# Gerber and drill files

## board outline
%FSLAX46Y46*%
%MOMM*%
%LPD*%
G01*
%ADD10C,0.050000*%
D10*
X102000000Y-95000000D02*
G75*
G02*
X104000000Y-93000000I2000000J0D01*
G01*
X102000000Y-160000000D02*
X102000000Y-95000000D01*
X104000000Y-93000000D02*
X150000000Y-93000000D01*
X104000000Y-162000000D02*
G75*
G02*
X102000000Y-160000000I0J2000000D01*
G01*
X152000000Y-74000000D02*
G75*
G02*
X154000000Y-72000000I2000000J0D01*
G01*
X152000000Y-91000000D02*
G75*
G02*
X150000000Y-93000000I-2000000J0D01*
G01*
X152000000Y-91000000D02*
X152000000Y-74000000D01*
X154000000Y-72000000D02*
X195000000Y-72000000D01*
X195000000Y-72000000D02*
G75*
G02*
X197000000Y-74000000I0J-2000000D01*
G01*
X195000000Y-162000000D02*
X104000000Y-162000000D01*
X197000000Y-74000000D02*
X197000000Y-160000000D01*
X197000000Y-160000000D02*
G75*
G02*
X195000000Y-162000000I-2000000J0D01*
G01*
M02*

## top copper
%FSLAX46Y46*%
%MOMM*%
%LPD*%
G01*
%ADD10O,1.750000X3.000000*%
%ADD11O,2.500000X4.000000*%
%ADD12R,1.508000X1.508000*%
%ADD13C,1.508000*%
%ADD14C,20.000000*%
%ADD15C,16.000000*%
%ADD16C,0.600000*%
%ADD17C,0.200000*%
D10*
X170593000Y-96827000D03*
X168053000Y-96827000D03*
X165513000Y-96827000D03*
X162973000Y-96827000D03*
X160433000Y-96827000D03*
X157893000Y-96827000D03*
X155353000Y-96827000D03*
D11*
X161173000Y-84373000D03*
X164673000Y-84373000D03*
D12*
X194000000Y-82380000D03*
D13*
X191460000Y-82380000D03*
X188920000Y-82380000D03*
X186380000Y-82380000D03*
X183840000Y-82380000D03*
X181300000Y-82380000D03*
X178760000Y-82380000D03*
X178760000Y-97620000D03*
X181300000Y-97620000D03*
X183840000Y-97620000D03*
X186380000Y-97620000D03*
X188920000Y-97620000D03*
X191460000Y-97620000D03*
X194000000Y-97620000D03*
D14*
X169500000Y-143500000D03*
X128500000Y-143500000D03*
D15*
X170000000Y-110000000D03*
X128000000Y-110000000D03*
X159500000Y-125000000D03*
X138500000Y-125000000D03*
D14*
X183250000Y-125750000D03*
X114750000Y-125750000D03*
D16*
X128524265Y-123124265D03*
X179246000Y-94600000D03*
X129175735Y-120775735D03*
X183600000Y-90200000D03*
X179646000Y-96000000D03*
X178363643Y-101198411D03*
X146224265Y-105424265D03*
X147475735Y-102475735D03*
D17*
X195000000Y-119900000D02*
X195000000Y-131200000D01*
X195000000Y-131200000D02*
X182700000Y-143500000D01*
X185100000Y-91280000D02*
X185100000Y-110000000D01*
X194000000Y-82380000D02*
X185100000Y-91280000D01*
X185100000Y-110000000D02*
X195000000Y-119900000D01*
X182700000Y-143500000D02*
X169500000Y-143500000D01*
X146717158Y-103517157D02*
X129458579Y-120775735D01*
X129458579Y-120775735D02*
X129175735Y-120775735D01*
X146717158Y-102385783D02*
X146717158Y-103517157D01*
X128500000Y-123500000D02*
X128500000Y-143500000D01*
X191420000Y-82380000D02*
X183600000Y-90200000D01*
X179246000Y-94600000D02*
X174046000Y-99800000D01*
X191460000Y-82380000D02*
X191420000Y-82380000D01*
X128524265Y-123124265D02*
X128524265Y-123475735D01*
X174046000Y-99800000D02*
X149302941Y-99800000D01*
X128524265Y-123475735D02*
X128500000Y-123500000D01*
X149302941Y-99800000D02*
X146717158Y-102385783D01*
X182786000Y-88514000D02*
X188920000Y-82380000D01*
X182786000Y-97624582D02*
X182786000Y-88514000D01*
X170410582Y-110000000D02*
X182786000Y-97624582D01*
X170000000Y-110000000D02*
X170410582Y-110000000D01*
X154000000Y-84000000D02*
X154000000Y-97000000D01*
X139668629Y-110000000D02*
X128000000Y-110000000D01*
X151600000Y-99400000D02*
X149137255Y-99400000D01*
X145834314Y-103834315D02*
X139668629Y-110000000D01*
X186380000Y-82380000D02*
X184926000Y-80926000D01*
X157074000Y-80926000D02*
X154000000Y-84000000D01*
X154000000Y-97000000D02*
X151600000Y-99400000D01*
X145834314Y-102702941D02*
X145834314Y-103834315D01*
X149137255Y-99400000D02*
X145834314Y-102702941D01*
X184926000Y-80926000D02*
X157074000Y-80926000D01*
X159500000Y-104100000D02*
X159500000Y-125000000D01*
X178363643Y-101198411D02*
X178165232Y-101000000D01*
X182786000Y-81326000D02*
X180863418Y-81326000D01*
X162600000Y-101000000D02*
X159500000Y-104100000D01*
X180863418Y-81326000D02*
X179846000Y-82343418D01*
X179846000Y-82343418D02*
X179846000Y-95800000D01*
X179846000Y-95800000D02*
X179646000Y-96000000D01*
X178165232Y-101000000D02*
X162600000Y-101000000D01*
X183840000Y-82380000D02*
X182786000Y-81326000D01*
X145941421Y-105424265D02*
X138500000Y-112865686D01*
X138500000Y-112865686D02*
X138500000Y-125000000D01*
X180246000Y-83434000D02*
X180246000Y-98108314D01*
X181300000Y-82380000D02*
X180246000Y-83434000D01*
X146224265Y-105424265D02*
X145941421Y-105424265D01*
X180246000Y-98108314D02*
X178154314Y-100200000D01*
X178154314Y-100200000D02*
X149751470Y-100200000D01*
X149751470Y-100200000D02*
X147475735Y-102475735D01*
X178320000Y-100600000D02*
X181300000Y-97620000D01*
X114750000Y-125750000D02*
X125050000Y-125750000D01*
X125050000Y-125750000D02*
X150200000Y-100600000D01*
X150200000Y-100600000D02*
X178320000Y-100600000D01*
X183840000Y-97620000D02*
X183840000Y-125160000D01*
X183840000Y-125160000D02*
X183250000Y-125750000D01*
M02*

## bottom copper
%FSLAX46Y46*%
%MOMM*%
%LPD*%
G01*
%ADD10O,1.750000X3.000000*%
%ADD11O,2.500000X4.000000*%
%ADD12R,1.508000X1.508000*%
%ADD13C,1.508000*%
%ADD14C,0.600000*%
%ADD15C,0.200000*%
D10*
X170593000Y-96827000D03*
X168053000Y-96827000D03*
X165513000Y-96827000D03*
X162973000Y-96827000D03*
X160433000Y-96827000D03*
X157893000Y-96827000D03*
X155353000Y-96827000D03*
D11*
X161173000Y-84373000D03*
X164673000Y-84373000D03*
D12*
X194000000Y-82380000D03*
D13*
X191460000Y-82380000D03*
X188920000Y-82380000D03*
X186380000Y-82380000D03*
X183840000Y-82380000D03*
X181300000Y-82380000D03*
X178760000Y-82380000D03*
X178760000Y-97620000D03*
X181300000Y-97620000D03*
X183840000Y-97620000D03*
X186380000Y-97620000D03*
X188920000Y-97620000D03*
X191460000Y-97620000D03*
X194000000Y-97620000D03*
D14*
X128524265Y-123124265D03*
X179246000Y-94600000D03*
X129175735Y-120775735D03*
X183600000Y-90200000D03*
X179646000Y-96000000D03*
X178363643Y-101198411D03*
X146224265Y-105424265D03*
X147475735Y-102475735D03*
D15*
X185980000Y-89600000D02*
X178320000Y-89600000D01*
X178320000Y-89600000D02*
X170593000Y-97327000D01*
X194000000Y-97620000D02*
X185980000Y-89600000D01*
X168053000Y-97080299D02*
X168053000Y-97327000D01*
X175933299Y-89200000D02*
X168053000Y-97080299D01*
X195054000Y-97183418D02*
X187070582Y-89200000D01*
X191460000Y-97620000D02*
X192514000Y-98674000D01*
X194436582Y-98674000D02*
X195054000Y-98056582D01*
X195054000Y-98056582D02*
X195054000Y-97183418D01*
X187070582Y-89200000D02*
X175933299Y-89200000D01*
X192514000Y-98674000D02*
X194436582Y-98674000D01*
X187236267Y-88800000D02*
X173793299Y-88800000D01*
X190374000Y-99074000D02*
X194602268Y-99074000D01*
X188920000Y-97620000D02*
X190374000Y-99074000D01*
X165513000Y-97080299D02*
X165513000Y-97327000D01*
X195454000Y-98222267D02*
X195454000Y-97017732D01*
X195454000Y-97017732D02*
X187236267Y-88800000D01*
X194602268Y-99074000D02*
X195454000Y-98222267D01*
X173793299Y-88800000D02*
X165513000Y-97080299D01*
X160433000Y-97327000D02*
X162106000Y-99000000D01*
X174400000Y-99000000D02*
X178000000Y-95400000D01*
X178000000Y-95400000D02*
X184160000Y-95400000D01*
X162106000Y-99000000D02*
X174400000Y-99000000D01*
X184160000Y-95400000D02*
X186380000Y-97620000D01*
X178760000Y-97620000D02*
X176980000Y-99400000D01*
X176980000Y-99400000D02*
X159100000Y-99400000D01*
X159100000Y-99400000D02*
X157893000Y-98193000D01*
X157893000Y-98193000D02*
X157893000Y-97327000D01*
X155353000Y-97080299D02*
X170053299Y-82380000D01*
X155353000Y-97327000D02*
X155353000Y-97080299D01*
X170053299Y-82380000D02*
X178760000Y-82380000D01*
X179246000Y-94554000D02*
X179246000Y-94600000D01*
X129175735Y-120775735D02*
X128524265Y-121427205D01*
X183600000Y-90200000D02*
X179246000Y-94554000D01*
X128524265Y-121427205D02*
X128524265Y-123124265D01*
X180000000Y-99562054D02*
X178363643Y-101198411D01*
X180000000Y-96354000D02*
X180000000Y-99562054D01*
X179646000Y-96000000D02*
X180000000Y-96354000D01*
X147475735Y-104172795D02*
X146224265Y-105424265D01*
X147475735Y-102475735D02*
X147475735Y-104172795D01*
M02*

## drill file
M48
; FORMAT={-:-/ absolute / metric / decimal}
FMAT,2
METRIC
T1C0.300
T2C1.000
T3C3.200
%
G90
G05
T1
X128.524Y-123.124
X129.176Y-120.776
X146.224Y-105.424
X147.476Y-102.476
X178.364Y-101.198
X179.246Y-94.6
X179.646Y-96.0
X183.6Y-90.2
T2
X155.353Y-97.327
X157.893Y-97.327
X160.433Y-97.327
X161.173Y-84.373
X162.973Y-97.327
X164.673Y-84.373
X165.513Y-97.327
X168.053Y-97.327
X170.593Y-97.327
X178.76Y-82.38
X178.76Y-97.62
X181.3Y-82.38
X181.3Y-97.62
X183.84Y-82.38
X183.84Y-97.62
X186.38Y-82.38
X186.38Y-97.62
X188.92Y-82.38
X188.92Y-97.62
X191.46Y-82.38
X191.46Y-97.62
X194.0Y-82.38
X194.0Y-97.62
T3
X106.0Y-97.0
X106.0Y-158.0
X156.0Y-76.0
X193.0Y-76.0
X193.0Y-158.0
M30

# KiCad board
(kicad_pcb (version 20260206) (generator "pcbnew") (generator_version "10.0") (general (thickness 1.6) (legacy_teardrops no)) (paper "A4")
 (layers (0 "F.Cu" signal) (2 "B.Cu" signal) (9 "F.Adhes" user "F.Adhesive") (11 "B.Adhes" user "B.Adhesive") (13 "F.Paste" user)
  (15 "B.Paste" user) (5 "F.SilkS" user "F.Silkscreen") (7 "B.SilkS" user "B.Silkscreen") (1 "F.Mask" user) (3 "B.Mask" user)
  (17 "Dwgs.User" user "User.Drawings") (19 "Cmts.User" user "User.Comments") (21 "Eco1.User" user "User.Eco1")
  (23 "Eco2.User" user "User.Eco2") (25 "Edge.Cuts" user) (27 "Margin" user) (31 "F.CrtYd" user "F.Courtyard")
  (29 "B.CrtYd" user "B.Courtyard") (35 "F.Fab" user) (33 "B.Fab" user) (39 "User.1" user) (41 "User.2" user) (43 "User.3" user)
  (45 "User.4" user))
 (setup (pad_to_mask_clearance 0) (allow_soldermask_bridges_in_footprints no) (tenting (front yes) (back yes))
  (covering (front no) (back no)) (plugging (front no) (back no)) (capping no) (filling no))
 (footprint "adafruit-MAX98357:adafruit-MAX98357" (layer "F.Cu") (at 163.093 90.42)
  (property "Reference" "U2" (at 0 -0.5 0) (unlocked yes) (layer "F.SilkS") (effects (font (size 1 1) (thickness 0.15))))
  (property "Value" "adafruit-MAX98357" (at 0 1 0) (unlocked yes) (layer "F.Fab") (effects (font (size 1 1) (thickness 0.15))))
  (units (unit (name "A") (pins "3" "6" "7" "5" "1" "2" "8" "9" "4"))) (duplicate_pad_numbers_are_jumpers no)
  (pad "1" thru_hole oval (at 7.5 6.907 270) (size 3 1.75) (drill 1 (offset -0.5 0)) (layers "*.Cu" "*.Mask") (remove_unused_layers no)
   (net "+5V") (solder_mask_margin 0.0508))
  (pad "2" thru_hole oval (at 4.96 6.907 270) (size 3 1.75) (drill 1 (offset -0.5 0)) (layers "*.Cu" "*.Mask") (remove_unused_layers no)
   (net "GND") (solder_mask_margin 0.0508))
  (pad "3" thru_hole oval (at 2.42 6.907 270) (size 3 1.75) (drill 1 (offset -0.5 0)) (layers "*.Cu" "*.Mask") (remove_unused_layers no)
   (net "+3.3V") (solder_mask_margin 0.0508))
  (pad "4" thru_hole oval (at -0.12 6.907 270) (size 3 1.75) (drill 1 (offset -0.5 0)) (layers "*.Cu" "*.Mask") (remove_unused_layers no)
   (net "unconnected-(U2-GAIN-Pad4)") (solder_mask_margin 0.0508))
  (pad "5" thru_hole oval (at -2.66 6.907 270) (size 3 1.75) (drill 1 (offset -0.5 0)) (layers "*.Cu" "*.Mask") (remove_unused_layers no)
   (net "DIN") (solder_mask_margin 0.0508))
  (pad "6" thru_hole oval (at -5.2 6.907 270) (size 3 1.75) (drill 1 (offset -0.5 0)) (layers "*.Cu" "*.Mask") (remove_unused_layers no)
   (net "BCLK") (solder_mask_margin 0.0508))
  (pad "7" thru_hole oval (at -7.74 6.907 270) (size 3 1.75) (drill 1 (offset -0.5 0)) (layers "*.Cu" "*.Mask") (remove_unused_layers no)
   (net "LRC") (solder_mask_margin 0.0508))
  (pad "8" thru_hole oval (at -1.92 -6.047 180) (size 2.5 4) (drill 1) (layers "*.Cu" "*.Mask") (remove_unused_layers no)
   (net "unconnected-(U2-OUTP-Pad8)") (solder_mask_margin 0.0508))
  (pad "9" thru_hole oval (at 1.58 -6.047 180) (size 2.5 4) (drill 1) (layers "*.Cu" "*.Mask") (remove_unused_layers no)
   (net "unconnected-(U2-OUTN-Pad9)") (solder_mask_margin 0.0508)))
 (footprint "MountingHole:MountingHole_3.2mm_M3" (layer "F.Cu") (at 106 158)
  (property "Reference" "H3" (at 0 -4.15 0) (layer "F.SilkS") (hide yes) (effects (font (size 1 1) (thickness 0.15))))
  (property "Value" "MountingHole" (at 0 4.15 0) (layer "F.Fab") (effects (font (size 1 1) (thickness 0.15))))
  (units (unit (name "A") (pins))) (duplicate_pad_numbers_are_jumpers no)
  (pad "" np_thru_hole circle (at 0 0) (size 3.2 3.2) (drill 3.2) (layers "*.Cu" "*.Mask")))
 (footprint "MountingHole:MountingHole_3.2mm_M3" (layer "F.Cu") (at 106 97)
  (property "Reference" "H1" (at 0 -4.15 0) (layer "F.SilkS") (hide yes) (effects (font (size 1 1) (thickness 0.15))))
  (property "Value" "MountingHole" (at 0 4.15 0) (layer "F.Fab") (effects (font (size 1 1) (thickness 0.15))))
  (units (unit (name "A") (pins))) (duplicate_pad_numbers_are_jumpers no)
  (pad "" np_thru_hole circle (at 0 0) (size 3.2 3.2) (drill 3.2) (layers "*.Cu" "*.Mask")))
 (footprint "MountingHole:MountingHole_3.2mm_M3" (layer "F.Cu") (at 156 76)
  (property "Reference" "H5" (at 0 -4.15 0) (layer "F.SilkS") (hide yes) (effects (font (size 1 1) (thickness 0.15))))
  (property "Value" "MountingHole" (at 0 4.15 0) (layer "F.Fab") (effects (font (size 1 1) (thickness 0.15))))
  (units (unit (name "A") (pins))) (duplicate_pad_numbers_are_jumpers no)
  (pad "" np_thru_hole circle (at 0 0) (size 3.2 3.2) (drill 3.2) (layers "*.Cu" "*.Mask")))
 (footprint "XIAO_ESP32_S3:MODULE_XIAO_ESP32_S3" (layer "F.Cu") (at 186.4435 90 -90)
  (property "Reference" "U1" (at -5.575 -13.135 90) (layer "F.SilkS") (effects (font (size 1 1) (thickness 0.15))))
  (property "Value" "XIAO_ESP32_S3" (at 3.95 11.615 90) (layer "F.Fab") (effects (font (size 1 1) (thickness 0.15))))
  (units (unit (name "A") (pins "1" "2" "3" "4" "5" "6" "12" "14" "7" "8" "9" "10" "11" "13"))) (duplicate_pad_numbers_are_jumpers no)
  (pad "1" thru_hole rect (at -7.62 -7.5565 270) (size 1.508 1.508) (drill 1) (layers "*.Cu" "*.Mask") (remove_unused_layers no)
   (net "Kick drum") (solder_mask_margin 0.102))
  (pad "2" thru_hole circle (at -7.62 -5.0165 270) (size 1.508 1.508) (drill 1) (layers "*.Cu" "*.Mask") (remove_unused_layers no)
   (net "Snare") (solder_mask_margin 0.102))
  (pad "3" thru_hole circle (at -7.62 -2.4765 270) (size 1.508 1.508) (drill 1) (layers "*.Cu" "*.Mask") (remove_unused_layers no)
   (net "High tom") (solder_mask_margin 0.102))
  (pad "4" thru_hole circle (at -7.62 0.0635 270) (size 1.508 1.508) (drill 1) (layers "*.Cu" "*.Mask") (remove_unused_layers no)
   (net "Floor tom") (solder_mask_margin 0.102))
  (pad "5" thru_hole circle (at -7.62 2.6035 270) (size 1.508 1.508) (drill 1) (layers "*.Cu" "*.Mask") (remove_unused_layers no)
   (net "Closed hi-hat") (solder_mask_margin 0.102))
  (pad "6" thru_hole circle (at -7.62 5.1435 270) (size 1.508 1.508) (drill 1) (layers "*.Cu" "*.Mask") (remove_unused_layers no)
   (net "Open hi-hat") (solder_mask_margin 0.102))
  (pad "7" thru_hole circle (at -7.62 7.6835 270) (size 1.508 1.508) (drill 1) (layers "*.Cu" "*.Mask") (remove_unused_layers no)
   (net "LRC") (solder_mask_margin 0.102))
  (pad "8" thru_hole circle (at 7.62 7.6835 270) (size 1.508 1.508) (drill 1) (layers "*.Cu" "*.Mask") (remove_unused_layers no)
   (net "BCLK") (solder_mask_margin 0.102))
  (pad "9" thru_hole circle (at 7.62 5.1435 270) (size 1.508 1.508) (drill 1) (layers "*.Cu" "*.Mask") (remove_unused_layers no)
   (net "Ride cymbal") (solder_mask_margin 0.102))
  (pad "10" thru_hole circle (at 7.62 2.6035 270) (size 1.508 1.508) (drill 1) (layers "*.Cu" "*.Mask") (remove_unused_layers no)
   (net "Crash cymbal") (solder_mask_margin 0.102))
  (pad "11" thru_hole circle (at 7.62 0.0635 270) (size 1.508 1.508) (drill 1) (layers "*.Cu" "*.Mask") (remove_unused_layers no)
   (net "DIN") (solder_mask_margin 0.102))
  (pad "12" thru_hole circle (at 7.62 -2.4765 270) (size 1.508 1.508) (drill 1) (layers "*.Cu" "*.Mask") (remove_unused_layers no)
   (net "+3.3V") (solder_mask_margin 0.102))
  (pad "13" thru_hole circle (at 7.62 -5.0165 270) (size 1.508 1.508) (drill 1) (layers "*.Cu" "*.Mask") (remove_unused_layers no)
   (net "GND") (solder_mask_margin 0.102))
  (pad "14" thru_hole circle (at 7.62 -7.5565 270) (size 1.508 1.508) (drill 1) (layers "*.Cu" "*.Mask") (remove_unused_layers no)
   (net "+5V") (solder_mask_margin 0.102)))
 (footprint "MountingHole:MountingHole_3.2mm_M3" (layer "F.Cu") (at 193 158)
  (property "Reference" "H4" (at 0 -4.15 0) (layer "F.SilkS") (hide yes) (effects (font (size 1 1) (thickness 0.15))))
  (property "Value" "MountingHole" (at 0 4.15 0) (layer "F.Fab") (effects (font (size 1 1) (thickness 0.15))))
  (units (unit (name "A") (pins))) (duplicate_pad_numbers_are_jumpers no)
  (pad "" np_thru_hole circle (at 0 0) (size 3.2 3.2) (drill 3.2) (layers "*.Cu" "*.Mask")))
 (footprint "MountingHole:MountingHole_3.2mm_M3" (layer "F.Cu") (at 193 76)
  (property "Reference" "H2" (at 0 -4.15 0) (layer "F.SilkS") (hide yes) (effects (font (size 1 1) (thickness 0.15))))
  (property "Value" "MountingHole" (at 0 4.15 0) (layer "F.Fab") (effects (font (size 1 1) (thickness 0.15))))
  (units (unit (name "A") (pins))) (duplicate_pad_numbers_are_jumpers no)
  (pad "" np_thru_hole circle (at 0 0) (size 3.2 3.2) (drill 3.2) (layers "*.Cu" "*.Mask")))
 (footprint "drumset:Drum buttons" (layer "F.Cu") (at 149 156)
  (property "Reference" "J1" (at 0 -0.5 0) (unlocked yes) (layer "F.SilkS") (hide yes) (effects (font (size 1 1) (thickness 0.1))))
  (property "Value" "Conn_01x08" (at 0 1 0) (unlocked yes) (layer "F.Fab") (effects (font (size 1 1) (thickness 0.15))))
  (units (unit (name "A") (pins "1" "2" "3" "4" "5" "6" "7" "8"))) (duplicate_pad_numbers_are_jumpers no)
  (pad "1" smd circle (at 20.5 -12.5) (size 20 20) (layers "F.Cu" "F.Mask") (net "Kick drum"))
  (pad "2" smd circle (at -20.5 -12.5) (size 20 20) (layers "F.Cu" "F.Mask") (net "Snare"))
  (pad "3" smd circle (at 21 -46) (size 16 16) (layers "F.Cu" "F.Mask") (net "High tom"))
  (pad "4" smd circle (at -21 -46) (size 16 16) (layers "F.Cu" "F.Mask") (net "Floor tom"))
  (pad "5" smd circle (at 10.5 -31) (size 16 16) (layers "F.Cu" "F.Mask") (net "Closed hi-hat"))
  (pad "6" smd circle (at -10.5 -31) (size 16 16) (layers "F.Cu" "F.Mask") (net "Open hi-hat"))
  (pad "7" smd circle (at 34.25 -30.25) (size 20 20) (layers "F.Cu" "F.Mask") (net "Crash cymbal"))
  (pad "8" smd circle (at -34.25 -30.25 90) (size 20 20) (layers "F.Cu" "F.Mask") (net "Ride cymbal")))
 (gr_arc (start 102 95) (mid 102.585786 93.585786) (end 104 93) (stroke (width 0.05) (type default)) (layer "Edge.Cuts"))
 (gr_line (start 102 160) (end 102 95) (stroke (width 0.05) (type default)) (layer "Edge.Cuts"))
 (gr_line (start 104 93) (end 150 93) (stroke (width 0.05) (type default)) (layer "Edge.Cuts"))
 (gr_arc (start 104 162) (mid 102.585786 161.414214) (end 102 160) (stroke (width 0.05) (type default)) (layer "Edge.Cuts"))
 (gr_arc (start 152 74) (mid 152.585786 72.585786) (end 154 72) (stroke (width 0.05) (type default)) (layer "Edge.Cuts"))
 (gr_arc (start 152 91) (mid 151.414214 92.414214) (end 150 93) (stroke (width 0.05) (type default)) (layer "Edge.Cuts"))
 (gr_line (start 152 91) (end 152 74) (stroke (width 0.05) (type default)) (layer "Edge.Cuts"))
 (gr_line (start 154 72) (end 195 72) (stroke (width 0.05) (type default)) (layer "Edge.Cuts"))
 (gr_arc (start 195 72) (mid 196.414214 72.585786) (end 197 74) (stroke (width 0.05) (type default)) (layer "Edge.Cuts"))
 (gr_line (start 195 162) (end 104 162) (stroke (width 0.05) (type default)) (layer "Edge.Cuts"))
 (gr_line (start 197 74) (end 197 160) (stroke (width 0.05) (type default)) (layer "Edge.Cuts"))
 (gr_arc (start 197 160) (mid 196.414214 161.414214) (end 195 162) (stroke (width 0.05) (type default)) (layer "Edge.Cuts"))
 (segment (start 185.98 89.6) (end 178.32 89.6) (width 0.2) (layer "B.Cu") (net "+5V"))
 (segment (start 178.32 89.6) (end 170.593 97.327) (width 0.2) (layer "B.Cu") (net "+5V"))
 (segment (start 194 97.62) (end 185.98 89.6) (width 0.2) (layer "B.Cu") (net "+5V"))
 (segment (start 168.053 97.080299) (end 168.053 97.327) (width 0.2) (layer "B.Cu") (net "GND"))
 (segment (start 175.933299 89.2) (end 168.053 97.080299) (width 0.2) (layer "B.Cu") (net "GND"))
 (segment (start 195.054 97.183418) (end 187.070582 89.2) (width 0.2) (layer "B.Cu") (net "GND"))
 (segment (start 191.46 97.62) (end 192.514 98.674) (width 0.2) (layer "B.Cu") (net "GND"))
 (segment (start 194.436582 98.674) (end 195.054 98.056582) (width 0.2) (layer "B.Cu") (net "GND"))
 (segment (start 195.054 98.056582) (end 195.054 97.183418) (width 0.2) (layer "B.Cu") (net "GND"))
 (segment (start 187.070582 89.2) (end 175.933299 89.2) (width 0.2) (layer "B.Cu") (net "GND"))
 (segment (start 192.514 98.674) (end 194.436582 98.674) (width 0.2) (layer "B.Cu") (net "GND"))
 (segment (start 187.236267 88.8) (end 173.793299 88.8) (width 0.2) (layer "B.Cu") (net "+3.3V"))
 (segment (start 190.374 99.074) (end 194.602268 99.074) (width 0.2) (layer "B.Cu") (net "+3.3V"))
 (segment (start 188.92 97.62) (end 190.374 99.074) (width 0.2) (layer "B.Cu") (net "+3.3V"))
 (segment (start 165.513 97.080299) (end 165.513 97.327) (width 0.2) (layer "B.Cu") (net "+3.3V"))
 (segment (start 195.454 98.222267) (end 195.454 97.017732) (width 0.2) (layer "B.Cu") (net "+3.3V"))
 (segment (start 195.454 97.017732) (end 187.236267 88.8) (width 0.2) (layer "B.Cu") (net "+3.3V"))
 (segment (start 194.602268 99.074) (end 195.454 98.222267) (width 0.2) (layer "B.Cu") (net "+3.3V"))
 (segment (start 173.793299 88.8) (end 165.513 97.080299) (width 0.2) (layer "B.Cu") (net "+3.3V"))
 (segment (start 160.433 97.327) (end 162.106 99) (width 0.2) (layer "B.Cu") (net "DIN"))
 (segment (start 174.4 99) (end 178 95.4) (width 0.2) (layer "B.Cu") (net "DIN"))
 (segment (start 178 95.4) (end 184.16 95.4) (width 0.2) (layer "B.Cu") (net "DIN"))
 (segment (start 162.106 99) (end 174.4 99) (width 0.2) (layer "B.Cu") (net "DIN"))
 (segment (start 184.16 95.4) (end 186.38 97.62) (width 0.2) (layer "B.Cu") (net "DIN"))
 (segment (start 178.76 97.62) (end 176.98 99.4) (width 0.2) (layer "B.Cu") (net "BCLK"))
 (segment (start 176.98 99.4) (end 159.1 99.4) (width 0.2) (layer "B.Cu") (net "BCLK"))
 (segment (start 159.1 99.4) (end 157.893 98.193) (width 0.2) (layer "B.Cu") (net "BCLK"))
 (segment (start 157.893 98.193) (end 157.893 97.327) (width 0.2) (layer "B.Cu") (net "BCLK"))
 (segment (start 155.353 97.080299) (end 170.053299 82.38) (width 0.2) (layer "B.Cu") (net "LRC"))
 (segment (start 155.353 97.327) (end 155.353 97.080299) (width 0.2) (layer "B.Cu") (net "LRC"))
 (segment (start 170.053299 82.38) (end 178.76 82.38) (width 0.2) (layer "B.Cu") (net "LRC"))
 (segment (start 195 119.9) (end 195 131.2) (width 0.2) (layer "F.Cu") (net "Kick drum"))
 (segment (start 195 131.2) (end 182.7 143.5) (width 0.2) (layer "F.Cu") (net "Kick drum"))
 (segment (start 185.1 91.28) (end 185.1 110) (width 0.2) (layer "F.Cu") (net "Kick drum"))
 (segment (start 194 82.38) (end 185.1 91.28) (width 0.2) (layer "F.Cu") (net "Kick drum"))
 (segment (start 185.1 110) (end 195 119.9) (width 0.2) (layer "F.Cu") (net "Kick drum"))
 (segment (start 182.7 143.5) (end 169.5 143.5) (width 0.2) (layer "F.Cu") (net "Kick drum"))
 (segment (start 146.717158 103.517157) (end 129.458579 120.775735) (width 0.2) (layer "F.Cu") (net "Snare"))
 (segment (start 129.458579 120.775735) (end 129.175735 120.775735) (width 0.2) (layer "F.Cu") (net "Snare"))
 (segment (start 146.717158 102.385783) (end 146.717158 103.517157) (width 0.2) (layer "F.Cu") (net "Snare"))
 (segment (start 128.5 123.5) (end 128.5 143.5) (width 0.2) (layer "F.Cu") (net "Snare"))
 (segment (start 191.42 82.38) (end 183.6 90.2) (width 0.2) (layer "F.Cu") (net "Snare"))
 (segment (start 179.246 94.6) (end 174.046 99.8) (width 0.2) (layer "F.Cu") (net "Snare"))
 (segment (start 191.46 82.38) (end 191.42 82.38) (width 0.2) (layer "F.Cu") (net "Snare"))
 (segment (start 128.524265 123.124265) (end 128.524265 123.475735) (width 0.2) (layer "F.Cu") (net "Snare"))
 (segment (start 174.046 99.8) (end 149.302941 99.8) (width 0.2) (layer "F.Cu") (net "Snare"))
 (segment (start 128.524265 123.475735) (end 128.5 123.5) (width 0.2) (layer "F.Cu") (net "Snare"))
 (segment (start 149.302941 99.8) (end 146.717158 102.385783) (width 0.2) (layer "F.Cu") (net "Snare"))
 (via (at 128.524265 123.124265) (size 0.6) (drill 0.3) (layers "F.Cu" "B.Cu") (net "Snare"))
 (via (at 179.246 94.6) (size 0.6) (drill 0.3) (layers "F.Cu" "B.Cu") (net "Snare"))
 (via (at 129.175735 120.775735) (size 0.6) (drill 0.3) (layers "F.Cu" "B.Cu") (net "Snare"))
 (via (at 183.6 90.2) (size 0.6) (drill 0.3) (layers "F.Cu" "B.Cu") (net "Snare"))
 (segment (start 179.246 94.554) (end 179.246 94.6) (width 0.2) (layer "B.Cu") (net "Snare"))
 (segment (start 129.175735 120.775735) (end 128.524265 121.427205) (width 0.2) (layer "B.Cu") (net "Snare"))
 (segment (start 183.6 90.2) (end 179.246 94.554) (width 0.2) (layer "B.Cu") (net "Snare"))
 (segment (start 128.524265 121.427205) (end 128.524265 123.124265) (width 0.2) (layer "B.Cu") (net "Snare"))
 (segment (start 182.786 88.514) (end 188.92 82.38) (width 0.2) (layer "F.Cu") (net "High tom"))
 (segment (start 182.786 97.624582) (end 182.786 88.514) (width 0.2) (layer "F.Cu") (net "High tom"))
 (segment (start 170.410582 110) (end 182.786 97.624582) (width 0.2) (layer "F.Cu") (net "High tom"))
 (segment (start 170 110) (end 170.410582 110) (width 0.2) (layer "F.Cu") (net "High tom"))
 (segment (start 154 84) (end 154 97) (width 0.2) (layer "F.Cu") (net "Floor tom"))
 (segment (start 139.668629 110) (end 128 110) (width 0.2) (layer "F.Cu") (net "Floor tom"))
 (segment (start 151.6 99.4) (end 149.137255 99.4) (width 0.2) (layer "F.Cu") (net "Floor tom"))
 (segment (start 145.834314 103.834315) (end 139.668629 110) (width 0.2) (layer "F.Cu") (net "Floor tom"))
 (segment (start 186.38 82.38) (end 184.926 80.926) (width 0.2) (layer "F.Cu") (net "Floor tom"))
 (segment (start 157.074 80.926) (end 154 84) (width 0.2) (layer "F.Cu") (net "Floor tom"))
 (segment (start 154 97) (end 151.6 99.4) (width 0.2) (layer "F.Cu") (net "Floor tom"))
 (segment (start 145.834314 102.702941) (end 145.834314 103.834315) (width 0.2) (layer "F.Cu") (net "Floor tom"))
 (segment (start 149.137255 99.4) (end 145.834314 102.702941) (width 0.2) (layer "F.Cu") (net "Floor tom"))
 (segment (start 184.926 80.926) (end 157.074 80.926) (width 0.2) (layer "F.Cu") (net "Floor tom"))
 (segment (start 159.5 104.1) (end 159.5 125) (width 0.2) (layer "F.Cu") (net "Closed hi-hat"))
 (segment (start 178.363643 101.198411) (end 178.165232 101) (width 0.2) (layer "F.Cu") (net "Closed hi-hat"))
 (segment (start 182.786 81.326) (end 180.863418 81.326) (width 0.2) (layer "F.Cu") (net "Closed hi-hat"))
 (segment (start 162.6 101) (end 159.5 104.1) (width 0.2) (layer "F.Cu") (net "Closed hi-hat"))
 (segment (start 180.863418 81.326) (end 179.846 82.343418) (width 0.2) (layer "F.Cu") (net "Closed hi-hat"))
 (segment (start 179.846 82.343418) (end 179.846 95.8) (width 0.2) (layer "F.Cu") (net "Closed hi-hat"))
 (segment (start 179.846 95.8) (end 179.646 96) (width 0.2) (layer "F.Cu") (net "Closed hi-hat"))
 (segment (start 178.165232 101) (end 162.6 101) (width 0.2) (layer "F.Cu") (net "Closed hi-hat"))
 (segment (start 183.84 82.38) (end 182.786 81.326) (width 0.2) (layer "F.Cu") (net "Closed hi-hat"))
 (via (at 179.646 96) (size 0.6) (drill 0.3) (layers "F.Cu" "B.Cu") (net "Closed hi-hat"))
 (via (at 178.363643 101.198411) (size 0.6) (drill 0.3) (layers "F.Cu" "B.Cu") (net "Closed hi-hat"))
 (segment (start 180 99.562054) (end 178.363643 101.198411) (width 0.2) (layer "B.Cu") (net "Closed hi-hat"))
 (segment (start 180 96.354) (end 180 99.562054) (width 0.2) (layer "B.Cu") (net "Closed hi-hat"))
 (segment (start 179.646 96) (end 180 96.354) (width 0.2) (layer "B.Cu") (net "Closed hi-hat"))
 (segment (start 145.941421 105.424265) (end 138.5 112.865686) (width 0.2) (layer "F.Cu") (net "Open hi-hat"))
 (segment (start 138.5 112.865686) (end 138.5 125) (width 0.2) (layer "F.Cu") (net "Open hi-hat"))
 (segment (start 180.246 83.434) (end 180.246 98.108314) (width 0.2) (layer "F.Cu") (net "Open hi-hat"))
 (segment (start 181.3 82.38) (end 180.246 83.434) (width 0.2) (layer "F.Cu") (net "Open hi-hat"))
 (segment (start 146.224265 105.424265) (end 145.941421 105.424265) (width 0.2) (layer "F.Cu") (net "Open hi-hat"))
 (segment (start 180.246 98.108314) (end 178.154314 100.2) (width 0.2) (layer "F.Cu") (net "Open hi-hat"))
 (segment (start 178.154314 100.2) (end 149.75147 100.2) (width 0.2) (layer "F.Cu") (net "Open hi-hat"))
 (segment (start 149.75147 100.2) (end 147.475735 102.475735) (width 0.2) (layer "F.Cu") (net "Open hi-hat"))
 (via (at 146.224265 105.424265) (size 0.6) (drill 0.3) (layers "F.Cu" "B.Cu") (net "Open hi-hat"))
 (via (at 147.475735 102.475735) (size 0.6) (drill 0.3) (layers "F.Cu" "B.Cu") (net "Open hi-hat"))
 (segment (start 147.475735 104.172795) (end 146.224265 105.424265) (width 0.2) (layer "B.Cu") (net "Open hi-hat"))
 (segment (start 147.475735 102.475735) (end 147.475735 104.172795) (width 0.2) (layer "B.Cu") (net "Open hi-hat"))
 (segment (start 178.32 100.6) (end 181.3 97.62) (width 0.2) (layer "F.Cu") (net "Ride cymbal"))
 (segment (start 114.75 125.75) (end 125.05 125.75) (width 0.2) (layer "F.Cu") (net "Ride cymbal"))
 (segment (start 125.05 125.75) (end 150.2 100.6) (width 0.2) (layer "F.Cu") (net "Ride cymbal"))
 (segment (start 150.2 100.6) (end 178.32 100.6) (width 0.2) (layer "F.Cu") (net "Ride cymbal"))
 (segment (start 183.84 97.62) (end 183.84 125.16) (width 0.2) (layer "F.Cu") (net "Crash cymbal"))
 (segment (start 183.84 125.16) (end 183.25 125.75) (width 0.2) (layer "F.Cu") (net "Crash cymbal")))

